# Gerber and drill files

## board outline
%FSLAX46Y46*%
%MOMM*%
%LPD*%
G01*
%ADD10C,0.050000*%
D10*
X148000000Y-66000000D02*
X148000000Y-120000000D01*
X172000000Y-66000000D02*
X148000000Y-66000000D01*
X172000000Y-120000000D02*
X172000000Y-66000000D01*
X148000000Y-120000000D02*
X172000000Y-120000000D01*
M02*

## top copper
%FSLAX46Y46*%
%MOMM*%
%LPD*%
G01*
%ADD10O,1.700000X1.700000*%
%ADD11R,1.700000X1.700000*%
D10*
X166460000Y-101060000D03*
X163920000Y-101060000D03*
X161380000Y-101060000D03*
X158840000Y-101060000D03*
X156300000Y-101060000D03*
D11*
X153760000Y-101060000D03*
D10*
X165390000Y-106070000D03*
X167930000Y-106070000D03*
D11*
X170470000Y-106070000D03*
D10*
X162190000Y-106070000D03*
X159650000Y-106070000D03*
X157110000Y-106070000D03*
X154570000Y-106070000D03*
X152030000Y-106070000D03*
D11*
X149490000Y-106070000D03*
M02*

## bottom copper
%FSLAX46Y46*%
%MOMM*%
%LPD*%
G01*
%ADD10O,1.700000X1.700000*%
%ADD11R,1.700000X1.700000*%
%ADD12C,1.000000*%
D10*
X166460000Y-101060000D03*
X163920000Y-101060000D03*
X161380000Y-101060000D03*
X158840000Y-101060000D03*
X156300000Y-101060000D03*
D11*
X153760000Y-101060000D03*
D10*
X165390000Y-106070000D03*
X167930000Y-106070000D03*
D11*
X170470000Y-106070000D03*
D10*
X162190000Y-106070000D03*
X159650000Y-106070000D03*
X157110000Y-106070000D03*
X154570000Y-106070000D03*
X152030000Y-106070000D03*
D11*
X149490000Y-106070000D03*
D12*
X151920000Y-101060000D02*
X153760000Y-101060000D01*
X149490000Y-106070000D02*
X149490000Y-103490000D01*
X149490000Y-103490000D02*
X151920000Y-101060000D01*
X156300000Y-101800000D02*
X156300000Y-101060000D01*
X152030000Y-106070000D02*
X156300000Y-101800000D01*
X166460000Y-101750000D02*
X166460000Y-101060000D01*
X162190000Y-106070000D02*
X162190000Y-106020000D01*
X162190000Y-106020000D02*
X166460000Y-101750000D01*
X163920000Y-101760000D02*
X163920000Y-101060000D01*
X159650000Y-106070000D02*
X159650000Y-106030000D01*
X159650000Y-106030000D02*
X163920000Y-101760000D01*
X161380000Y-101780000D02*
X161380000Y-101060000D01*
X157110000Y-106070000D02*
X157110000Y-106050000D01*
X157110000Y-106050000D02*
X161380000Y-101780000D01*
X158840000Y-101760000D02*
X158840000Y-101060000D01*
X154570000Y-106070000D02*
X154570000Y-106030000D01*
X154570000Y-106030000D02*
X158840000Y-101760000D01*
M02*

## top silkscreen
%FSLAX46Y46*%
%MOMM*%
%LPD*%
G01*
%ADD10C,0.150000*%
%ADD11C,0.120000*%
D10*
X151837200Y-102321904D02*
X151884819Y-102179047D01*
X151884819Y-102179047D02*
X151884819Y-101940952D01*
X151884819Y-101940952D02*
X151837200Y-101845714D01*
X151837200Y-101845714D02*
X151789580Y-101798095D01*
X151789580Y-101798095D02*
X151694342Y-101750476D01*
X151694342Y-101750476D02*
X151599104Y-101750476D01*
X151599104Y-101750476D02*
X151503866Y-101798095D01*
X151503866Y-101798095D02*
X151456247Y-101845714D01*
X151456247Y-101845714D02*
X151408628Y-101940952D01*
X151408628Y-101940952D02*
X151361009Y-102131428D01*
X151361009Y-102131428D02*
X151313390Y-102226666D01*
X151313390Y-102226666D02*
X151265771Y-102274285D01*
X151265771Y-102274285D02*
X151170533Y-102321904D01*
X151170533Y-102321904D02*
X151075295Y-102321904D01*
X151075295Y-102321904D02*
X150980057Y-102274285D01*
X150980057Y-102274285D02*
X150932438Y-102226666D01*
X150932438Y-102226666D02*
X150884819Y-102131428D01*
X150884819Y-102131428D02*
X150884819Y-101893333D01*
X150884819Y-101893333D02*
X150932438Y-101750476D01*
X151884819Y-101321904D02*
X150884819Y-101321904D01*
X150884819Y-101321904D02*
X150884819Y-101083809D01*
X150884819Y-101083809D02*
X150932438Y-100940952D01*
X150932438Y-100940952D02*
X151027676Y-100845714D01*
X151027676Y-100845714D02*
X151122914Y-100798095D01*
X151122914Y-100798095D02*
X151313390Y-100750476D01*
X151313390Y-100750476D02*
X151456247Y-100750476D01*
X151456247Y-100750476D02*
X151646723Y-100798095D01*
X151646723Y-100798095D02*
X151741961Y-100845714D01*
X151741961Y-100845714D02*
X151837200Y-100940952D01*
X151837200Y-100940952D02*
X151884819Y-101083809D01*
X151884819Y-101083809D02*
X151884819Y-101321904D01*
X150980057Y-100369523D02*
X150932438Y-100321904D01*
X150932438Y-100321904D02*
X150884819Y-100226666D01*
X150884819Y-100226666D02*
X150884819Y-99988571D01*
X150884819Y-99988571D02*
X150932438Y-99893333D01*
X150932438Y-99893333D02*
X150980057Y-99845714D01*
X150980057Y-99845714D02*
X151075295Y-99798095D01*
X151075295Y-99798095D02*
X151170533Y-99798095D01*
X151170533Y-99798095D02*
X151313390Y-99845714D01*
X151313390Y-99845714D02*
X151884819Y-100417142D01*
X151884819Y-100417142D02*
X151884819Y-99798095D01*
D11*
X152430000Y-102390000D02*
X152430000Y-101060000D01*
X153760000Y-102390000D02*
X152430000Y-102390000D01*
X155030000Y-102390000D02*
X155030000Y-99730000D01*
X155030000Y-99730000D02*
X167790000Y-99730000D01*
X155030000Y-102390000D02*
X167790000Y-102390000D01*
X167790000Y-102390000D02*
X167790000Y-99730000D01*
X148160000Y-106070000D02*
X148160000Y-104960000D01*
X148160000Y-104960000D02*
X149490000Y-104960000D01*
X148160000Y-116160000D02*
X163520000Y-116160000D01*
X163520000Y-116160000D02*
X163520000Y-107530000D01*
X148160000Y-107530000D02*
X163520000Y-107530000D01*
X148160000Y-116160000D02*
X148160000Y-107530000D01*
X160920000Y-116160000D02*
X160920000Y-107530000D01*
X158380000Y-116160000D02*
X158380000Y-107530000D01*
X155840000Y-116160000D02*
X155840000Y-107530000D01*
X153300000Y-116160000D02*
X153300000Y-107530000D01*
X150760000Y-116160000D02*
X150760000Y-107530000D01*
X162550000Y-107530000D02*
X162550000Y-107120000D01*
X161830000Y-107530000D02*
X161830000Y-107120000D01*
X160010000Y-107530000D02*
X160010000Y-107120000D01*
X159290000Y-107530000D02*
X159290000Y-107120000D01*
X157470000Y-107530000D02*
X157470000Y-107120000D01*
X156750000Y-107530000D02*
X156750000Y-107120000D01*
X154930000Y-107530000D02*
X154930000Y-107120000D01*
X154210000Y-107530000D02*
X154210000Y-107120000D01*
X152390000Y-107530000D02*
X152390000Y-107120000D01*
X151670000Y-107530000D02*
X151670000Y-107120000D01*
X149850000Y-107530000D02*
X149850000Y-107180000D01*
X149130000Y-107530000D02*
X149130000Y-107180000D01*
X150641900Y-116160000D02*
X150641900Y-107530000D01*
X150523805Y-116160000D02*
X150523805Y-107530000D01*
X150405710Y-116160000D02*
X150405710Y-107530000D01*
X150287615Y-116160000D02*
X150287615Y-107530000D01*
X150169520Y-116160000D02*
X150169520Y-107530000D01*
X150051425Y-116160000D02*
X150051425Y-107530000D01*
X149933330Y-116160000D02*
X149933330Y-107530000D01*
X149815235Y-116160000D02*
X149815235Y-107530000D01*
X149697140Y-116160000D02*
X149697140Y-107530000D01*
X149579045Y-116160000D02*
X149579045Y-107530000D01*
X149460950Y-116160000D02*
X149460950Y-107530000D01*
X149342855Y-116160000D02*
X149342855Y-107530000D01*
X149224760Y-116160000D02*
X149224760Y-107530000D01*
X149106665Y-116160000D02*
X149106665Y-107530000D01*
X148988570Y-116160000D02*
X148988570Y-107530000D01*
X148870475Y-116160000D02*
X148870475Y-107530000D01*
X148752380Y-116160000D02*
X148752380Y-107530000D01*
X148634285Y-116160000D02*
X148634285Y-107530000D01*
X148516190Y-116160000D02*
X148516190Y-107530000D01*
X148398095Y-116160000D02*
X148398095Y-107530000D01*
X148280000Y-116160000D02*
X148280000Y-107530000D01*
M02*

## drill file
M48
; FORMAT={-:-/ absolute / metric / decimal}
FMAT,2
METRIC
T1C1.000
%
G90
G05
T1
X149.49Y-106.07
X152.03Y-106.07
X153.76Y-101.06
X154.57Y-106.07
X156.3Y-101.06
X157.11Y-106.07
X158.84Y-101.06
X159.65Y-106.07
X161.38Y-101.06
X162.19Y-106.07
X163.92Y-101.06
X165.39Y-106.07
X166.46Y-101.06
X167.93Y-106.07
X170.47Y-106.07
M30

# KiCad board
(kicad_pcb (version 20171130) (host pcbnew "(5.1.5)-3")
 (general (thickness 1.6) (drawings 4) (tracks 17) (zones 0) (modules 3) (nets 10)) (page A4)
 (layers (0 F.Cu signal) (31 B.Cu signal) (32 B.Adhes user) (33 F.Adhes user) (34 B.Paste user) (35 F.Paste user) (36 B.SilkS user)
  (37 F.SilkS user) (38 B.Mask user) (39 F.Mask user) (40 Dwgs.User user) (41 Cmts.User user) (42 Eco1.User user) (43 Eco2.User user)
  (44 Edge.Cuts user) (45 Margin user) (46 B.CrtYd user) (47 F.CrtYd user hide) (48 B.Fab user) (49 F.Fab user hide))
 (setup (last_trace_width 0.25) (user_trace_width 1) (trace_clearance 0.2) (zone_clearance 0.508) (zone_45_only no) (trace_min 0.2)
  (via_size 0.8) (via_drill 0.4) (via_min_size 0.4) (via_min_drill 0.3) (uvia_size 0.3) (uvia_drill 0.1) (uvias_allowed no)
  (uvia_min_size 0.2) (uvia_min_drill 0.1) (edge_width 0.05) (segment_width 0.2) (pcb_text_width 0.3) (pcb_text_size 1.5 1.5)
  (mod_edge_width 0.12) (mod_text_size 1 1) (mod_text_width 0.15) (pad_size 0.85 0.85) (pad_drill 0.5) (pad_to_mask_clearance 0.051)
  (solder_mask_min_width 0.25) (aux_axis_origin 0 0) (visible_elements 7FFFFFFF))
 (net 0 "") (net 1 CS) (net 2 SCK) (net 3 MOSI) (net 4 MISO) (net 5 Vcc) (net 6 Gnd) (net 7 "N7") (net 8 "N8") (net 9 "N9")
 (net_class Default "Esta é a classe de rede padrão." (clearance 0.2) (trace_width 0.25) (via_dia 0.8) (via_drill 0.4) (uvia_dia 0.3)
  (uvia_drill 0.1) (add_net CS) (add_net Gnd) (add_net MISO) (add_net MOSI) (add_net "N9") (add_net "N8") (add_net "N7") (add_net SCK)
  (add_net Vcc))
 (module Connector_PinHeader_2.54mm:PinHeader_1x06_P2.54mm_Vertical (layer F.Cu) (at 153.76 101.06 90)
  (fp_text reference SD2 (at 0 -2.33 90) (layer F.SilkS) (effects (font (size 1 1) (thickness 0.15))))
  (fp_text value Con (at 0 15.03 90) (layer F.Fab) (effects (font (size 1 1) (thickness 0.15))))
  (fp_line (start -1.33 -1.33) (end 0 -1.33) (layer F.SilkS) (width 0.12))
  (fp_line (start -1.33 0) (end -1.33 -1.33) (layer F.SilkS) (width 0.12))
  (fp_line (start -1.33 1.27) (end 1.33 1.27) (layer F.SilkS) (width 0.12))
  (fp_line (start 1.33 1.27) (end 1.33 14.03) (layer F.SilkS) (width 0.12))
  (fp_line (start -1.33 1.27) (end -1.33 14.03) (layer F.SilkS) (width 0.12))
  (fp_line (start -1.33 14.03) (end 1.33 14.03) (layer F.SilkS) (width 0.12))
  (pad 6 thru_hole oval (at 0 12.7 90) (size 1.7 1.7) (drill 1) (layers *.Cu *.Mask) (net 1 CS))
  (pad 5 thru_hole oval (at 0 10.16 90) (size 1.7 1.7) (drill 1) (layers *.Cu *.Mask) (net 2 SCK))
  (pad 4 thru_hole oval (at 0 7.62 90) (size 1.7 1.7) (drill 1) (layers *.Cu *.Mask) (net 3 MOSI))
  (pad 3 thru_hole oval (at 0 5.08 90) (size 1.7 1.7) (drill 1) (layers *.Cu *.Mask) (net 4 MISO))
  (pad 2 thru_hole oval (at 0 2.54 90) (size 1.7 1.7) (drill 1) (layers *.Cu *.Mask) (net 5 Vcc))
  (pad 1 thru_hole rect (at 0 0 90) (size 1.7 1.7) (drill 1) (layers *.Cu *.Mask) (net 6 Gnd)))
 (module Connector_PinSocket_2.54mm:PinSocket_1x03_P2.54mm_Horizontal (layer B.Cu) (at 170.47 106.07 90)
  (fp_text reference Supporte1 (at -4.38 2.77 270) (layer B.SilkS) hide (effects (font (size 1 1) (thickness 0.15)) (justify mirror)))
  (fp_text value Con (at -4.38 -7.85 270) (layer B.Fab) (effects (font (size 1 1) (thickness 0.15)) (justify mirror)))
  (pad 3 thru_hole oval (at 0 -5.08 90) (size 1.7 1.7) (drill 1) (layers *.Cu *.Mask) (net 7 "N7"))
  (pad 2 thru_hole oval (at 0 -2.54 90) (size 1.7 1.7) (drill 1) (layers *.Cu *.Mask) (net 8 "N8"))
  (pad 1 thru_hole rect (at 0 0 90) (size 1.7 1.7) (drill 1) (layers *.Cu *.Mask) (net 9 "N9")))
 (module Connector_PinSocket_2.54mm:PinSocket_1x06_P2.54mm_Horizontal (layer F.Cu) (at 149.49 106.07 90)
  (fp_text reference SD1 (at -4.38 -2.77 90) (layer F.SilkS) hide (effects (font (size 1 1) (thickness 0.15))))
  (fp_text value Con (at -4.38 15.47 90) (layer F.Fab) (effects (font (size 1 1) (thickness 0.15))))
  (fp_line (start 0 -1.33) (end 1.11 -1.33) (layer F.SilkS) (width 0.12))
  (fp_line (start 1.11 -1.33) (end 1.11 0) (layer F.SilkS) (width 0.12))
  (fp_line (start -10.09 -1.33) (end -10.09 14.03) (layer F.SilkS) (width 0.12))
  (fp_line (start -10.09 14.03) (end -1.46 14.03) (layer F.SilkS) (width 0.12))
  (fp_line (start -1.46 -1.33) (end -1.46 14.03) (layer F.SilkS) (width 0.12))
  (fp_line (start -10.09 -1.33) (end -1.46 -1.33) (layer F.SilkS) (width 0.12))
  (fp_line (start -10.09 11.43) (end -1.46 11.43) (layer F.SilkS) (width 0.12))
  (fp_line (start -10.09 8.89) (end -1.46 8.89) (layer F.SilkS) (width 0.12))
  (fp_line (start -10.09 6.35) (end -1.46 6.35) (layer F.SilkS) (width 0.12))
  (fp_line (start -10.09 3.81) (end -1.46 3.81) (layer F.SilkS) (width 0.12))
  (fp_line (start -10.09 1.27) (end -1.46 1.27) (layer F.SilkS) (width 0.12))
  (fp_line (start -1.46 13.06) (end -1.05 13.06) (layer F.SilkS) (width 0.12))
  (fp_line (start -1.46 12.34) (end -1.05 12.34) (layer F.SilkS) (width 0.12))
  (fp_line (start -1.46 10.52) (end -1.05 10.52) (layer F.SilkS) (width 0.12))
  (fp_line (start -1.46 9.8) (end -1.05 9.8) (layer F.SilkS) (width 0.12))
  (fp_line (start -1.46 7.98) (end -1.05 7.98) (layer F.SilkS) (width 0.12))
  (fp_line (start -1.46 7.26) (end -1.05 7.26) (layer F.SilkS) (width 0.12))
  (fp_line (start -1.46 5.44) (end -1.05 5.44) (layer F.SilkS) (width 0.12))
  (fp_line (start -1.46 4.72) (end -1.05 4.72) (layer F.SilkS) (width 0.12))
  (fp_line (start -1.46 2.9) (end -1.05 2.9) (layer F.SilkS) (width 0.12))
  (fp_line (start -1.46 2.18) (end -1.05 2.18) (layer F.SilkS) (width 0.12))
  (fp_line (start -1.46 0.36) (end -1.11 0.36) (layer F.SilkS) (width 0.12))
  (fp_line (start -1.46 -0.36) (end -1.11 -0.36) (layer F.SilkS) (width 0.12))
  (fp_line (start -10.09 1.1519) (end -1.46 1.1519) (layer F.SilkS) (width 0.12))
  (fp_line (start -10.09 1.033805) (end -1.46 1.033805) (layer F.SilkS) (width 0.12))
  (fp_line (start -10.09 0.91571) (end -1.46 0.91571) (layer F.SilkS) (width 0.12))
  (fp_line (start -10.09 0.797615) (end -1.46 0.797615) (layer F.SilkS) (width 0.12))
  (fp_line (start -10.09 0.67952) (end -1.46 0.67952) (layer F.SilkS) (width 0.12))
  (fp_line (start -10.09 0.561425) (end -1.46 0.561425) (layer F.SilkS) (width 0.12))
  (fp_line (start -10.09 0.44333) (end -1.46 0.44333) (layer F.SilkS) (width 0.12))
  (fp_line (start -10.09 0.325235) (end -1.46 0.325235) (layer F.SilkS) (width 0.12))
  (fp_line (start -10.09 0.20714) (end -1.46 0.20714) (layer F.SilkS) (width 0.12))
  (fp_line (start -10.09 0.089045) (end -1.46 0.089045) (layer F.SilkS) (width 0.12))
  (fp_line (start -10.09 -0.02905) (end -1.46 -0.02905) (layer F.SilkS) (width 0.12))
  (fp_line (start -10.09 -0.147145) (end -1.46 -0.147145) (layer F.SilkS) (width 0.12))
  (fp_line (start -10.09 -0.26524) (end -1.46 -0.26524) (layer F.SilkS) (width 0.12))
  (fp_line (start -10.09 -0.383335) (end -1.46 -0.383335) (layer F.SilkS) (width 0.12))
  (fp_line (start -10.09 -0.50143) (end -1.46 -0.50143) (layer F.SilkS) (width 0.12))
  (fp_line (start -10.09 -0.619525) (end -1.46 -0.619525) (layer F.SilkS) (width 0.12))
  (fp_line (start -10.09 -0.73762) (end -1.46 -0.73762) (layer F.SilkS) (width 0.12))
  (fp_line (start -10.09 -0.855715) (end -1.46 -0.855715) (layer F.SilkS) (width 0.12))
  (fp_line (start -10.09 -0.97381) (end -1.46 -0.97381) (layer F.SilkS) (width 0.12))
  (fp_line (start -10.09 -1.091905) (end -1.46 -1.091905) (layer F.SilkS) (width 0.12))
  (fp_line (start -10.09 -1.21) (end -1.46 -1.21) (layer F.SilkS) (width 0.12))
  (pad 6 thru_hole oval (at 0 12.7 90) (size 1.7 1.7) (drill 1) (layers *.Cu *.Mask) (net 1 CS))
  (pad 5 thru_hole oval (at 0 10.16 90) (size 1.7 1.7) (drill 1) (layers *.Cu *.Mask) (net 2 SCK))
  (pad 4 thru_hole oval (at 0 7.62 90) (size 1.7 1.7) (drill 1) (layers *.Cu *.Mask) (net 3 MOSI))
  (pad 3 thru_hole oval (at 0 5.08 90) (size 1.7 1.7) (drill 1) (layers *.Cu *.Mask) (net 4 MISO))
  (pad 2 thru_hole oval (at 0 2.54 90) (size 1.7 1.7) (drill 1) (layers *.Cu *.Mask) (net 5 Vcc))
  (pad 1 thru_hole rect (at 0 0 90) (size 1.7 1.7) (drill 1) (layers *.Cu *.Mask) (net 6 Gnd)))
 (gr_line (start 148 66) (end 148 120) (layer Edge.Cuts) (width 0.05))
 (gr_line (start 172 66) (end 148 66) (layer Edge.Cuts) (width 0.05))
 (gr_line (start 172 120) (end 172 66) (layer Edge.Cuts) (width 0.05))
 (gr_line (start 148 120) (end 172 120) (layer Edge.Cuts) (width 0.05))
 (segment (start 151.92 101.06) (end 153.76 101.06) (width 1) (layer B.Cu) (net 6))
 (segment (start 149.49 106.07) (end 149.49 103.49) (width 1) (layer B.Cu) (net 6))
 (segment (start 149.49 103.49) (end 151.92 101.06) (width 1) (layer B.Cu) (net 6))
 (segment (start 156.3 101.8) (end 156.3 101.06) (width 1) (layer B.Cu) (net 5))
 (segment (start 152.03 106.07) (end 156.3 101.8) (width 1) (layer B.Cu) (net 5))
 (segment (start 166.46 101.75) (end 166.46 101.06) (width 1) (layer B.Cu) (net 1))
 (segment (start 162.19 106.07) (end 162.19 106.02) (width 1) (layer B.Cu) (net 1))
 (segment (start 162.19 106.02) (end 166.46 101.75) (width 1) (layer B.Cu) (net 1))
 (segment (start 163.92 101.76) (end 163.92 101.06) (width 1) (layer B.Cu) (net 2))
 (segment (start 159.65 106.07) (end 159.65 106.03) (width 1) (layer B.Cu) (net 2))
 (segment (start 159.65 106.03) (end 163.92 101.76) (width 1) (layer B.Cu) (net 2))
 (segment (start 161.38 101.78) (end 161.38 101.06) (width 1) (layer B.Cu) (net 3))
 (segment (start 157.11 106.07) (end 157.11 106.05) (width 1) (layer B.Cu) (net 3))
 (segment (start 157.11 106.05) (end 161.38 101.78) (width 1) (layer B.Cu) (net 3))
 (segment (start 158.84 101.76) (end 158.84 101.06) (width 1) (layer B.Cu) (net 4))
 (segment (start 154.57 106.07) (end 154.57 106.03) (width 1) (layer B.Cu) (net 4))
 (segment (start 154.57 106.03) (end 158.84 101.76) (width 1) (layer B.Cu) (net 4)))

